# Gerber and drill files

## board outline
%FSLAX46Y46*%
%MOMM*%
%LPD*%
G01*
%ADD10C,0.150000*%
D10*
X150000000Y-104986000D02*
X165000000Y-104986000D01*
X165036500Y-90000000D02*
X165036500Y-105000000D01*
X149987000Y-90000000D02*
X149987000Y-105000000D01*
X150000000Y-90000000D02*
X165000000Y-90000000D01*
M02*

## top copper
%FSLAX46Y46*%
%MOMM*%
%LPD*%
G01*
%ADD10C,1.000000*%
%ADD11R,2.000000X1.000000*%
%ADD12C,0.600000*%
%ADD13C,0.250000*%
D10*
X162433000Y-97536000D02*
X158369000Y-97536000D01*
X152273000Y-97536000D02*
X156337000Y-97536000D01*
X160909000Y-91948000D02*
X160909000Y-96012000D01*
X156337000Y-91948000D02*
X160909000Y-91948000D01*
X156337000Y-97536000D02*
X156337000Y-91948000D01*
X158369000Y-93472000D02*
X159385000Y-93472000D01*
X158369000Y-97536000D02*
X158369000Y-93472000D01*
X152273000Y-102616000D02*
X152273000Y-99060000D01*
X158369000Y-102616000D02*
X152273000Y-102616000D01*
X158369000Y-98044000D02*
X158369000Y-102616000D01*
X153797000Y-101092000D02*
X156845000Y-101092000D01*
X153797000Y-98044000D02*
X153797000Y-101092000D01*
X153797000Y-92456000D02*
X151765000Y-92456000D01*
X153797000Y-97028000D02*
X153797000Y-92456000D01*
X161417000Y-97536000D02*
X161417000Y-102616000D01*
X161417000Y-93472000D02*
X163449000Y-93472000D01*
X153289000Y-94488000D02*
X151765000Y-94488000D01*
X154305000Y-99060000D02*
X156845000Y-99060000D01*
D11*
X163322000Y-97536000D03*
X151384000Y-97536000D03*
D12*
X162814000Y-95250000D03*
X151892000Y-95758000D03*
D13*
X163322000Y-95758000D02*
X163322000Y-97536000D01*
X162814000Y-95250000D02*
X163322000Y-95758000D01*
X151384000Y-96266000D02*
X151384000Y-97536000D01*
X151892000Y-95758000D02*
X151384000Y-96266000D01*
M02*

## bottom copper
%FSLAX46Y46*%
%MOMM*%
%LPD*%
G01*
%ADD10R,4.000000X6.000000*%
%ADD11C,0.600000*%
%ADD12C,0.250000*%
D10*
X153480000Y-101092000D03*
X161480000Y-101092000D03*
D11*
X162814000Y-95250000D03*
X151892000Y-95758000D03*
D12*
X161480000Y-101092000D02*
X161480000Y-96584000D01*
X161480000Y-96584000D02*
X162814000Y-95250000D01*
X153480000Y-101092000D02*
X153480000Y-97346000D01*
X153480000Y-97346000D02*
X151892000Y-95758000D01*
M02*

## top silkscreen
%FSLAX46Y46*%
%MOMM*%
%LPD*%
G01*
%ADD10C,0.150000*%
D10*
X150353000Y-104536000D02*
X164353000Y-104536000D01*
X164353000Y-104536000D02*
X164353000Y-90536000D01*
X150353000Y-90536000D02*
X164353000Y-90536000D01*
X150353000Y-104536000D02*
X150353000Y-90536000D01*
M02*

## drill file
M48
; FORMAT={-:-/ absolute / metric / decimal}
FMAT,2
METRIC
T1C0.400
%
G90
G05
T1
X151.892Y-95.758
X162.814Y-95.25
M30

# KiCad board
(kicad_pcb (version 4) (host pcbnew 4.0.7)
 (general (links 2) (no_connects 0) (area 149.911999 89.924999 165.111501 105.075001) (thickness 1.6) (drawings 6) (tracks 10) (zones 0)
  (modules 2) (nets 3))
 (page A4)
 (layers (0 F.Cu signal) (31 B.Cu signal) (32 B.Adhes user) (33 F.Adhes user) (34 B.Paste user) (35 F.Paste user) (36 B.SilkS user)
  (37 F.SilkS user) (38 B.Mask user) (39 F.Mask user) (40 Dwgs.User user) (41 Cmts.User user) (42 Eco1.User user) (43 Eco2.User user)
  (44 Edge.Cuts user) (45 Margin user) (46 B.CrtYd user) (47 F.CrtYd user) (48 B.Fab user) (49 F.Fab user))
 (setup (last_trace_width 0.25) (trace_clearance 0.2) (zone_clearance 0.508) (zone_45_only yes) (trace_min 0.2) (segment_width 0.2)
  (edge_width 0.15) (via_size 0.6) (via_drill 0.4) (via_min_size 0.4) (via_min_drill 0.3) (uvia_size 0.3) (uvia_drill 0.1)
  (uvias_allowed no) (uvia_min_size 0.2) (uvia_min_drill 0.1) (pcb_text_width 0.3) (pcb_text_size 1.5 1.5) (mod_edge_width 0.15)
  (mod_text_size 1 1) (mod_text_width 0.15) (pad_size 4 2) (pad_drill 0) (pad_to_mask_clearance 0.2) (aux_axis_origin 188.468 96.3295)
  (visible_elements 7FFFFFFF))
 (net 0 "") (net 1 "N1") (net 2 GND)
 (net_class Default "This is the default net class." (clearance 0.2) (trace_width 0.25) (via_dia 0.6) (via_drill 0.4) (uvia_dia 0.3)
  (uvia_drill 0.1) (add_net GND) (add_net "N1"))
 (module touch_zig (layer F.Cu) (at 157.353 97.536)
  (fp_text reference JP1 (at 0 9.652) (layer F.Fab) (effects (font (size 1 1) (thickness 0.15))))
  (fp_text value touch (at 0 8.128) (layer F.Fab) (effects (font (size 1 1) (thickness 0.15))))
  (fp_line (start 5.08 0) (end 1.016 0) (layer F.Cu) (width 1))
  (fp_line (start -5.08 0) (end -1.016 0) (layer F.Cu) (width 1))
  (fp_line (start 3.556 -5.588) (end 3.556 -1.524) (layer F.Cu) (width 1))
  (fp_line (start -1.016 -5.588) (end 3.556 -5.588) (layer F.Cu) (width 1))
  (fp_line (start -1.016 0) (end -1.016 -5.588) (layer F.Cu) (width 1))
  (fp_line (start 1.016 -4.064) (end 2.032 -4.064) (layer F.Cu) (width 1))
  (fp_line (start 1.016 0) (end 1.016 -4.064) (layer F.Cu) (width 1))
  (fp_line (start -5.08 5.08) (end -5.08 1.524) (layer F.Cu) (width 1))
  (fp_line (start 1.016 5.08) (end -5.08 5.08) (layer F.Cu) (width 1))
  (fp_line (start 1.016 0.508) (end 1.016 5.08) (layer F.Cu) (width 1))
  (fp_line (start -3.556 3.556) (end -0.508 3.556) (layer F.Cu) (width 1))
  (fp_line (start -3.556 0.508) (end -3.556 3.556) (layer F.Cu) (width 1))
  (fp_line (start -3.556 -5.08) (end -5.588 -5.08) (layer F.Cu) (width 1))
  (fp_line (start -3.556 -0.508) (end -3.556 -5.08) (layer F.Cu) (width 1))
  (fp_line (start 4.064 0) (end 4.064 5.08) (layer F.Cu) (width 1))
  (fp_line (start 4.064 -4.064) (end 6.096 -4.064) (layer F.Cu) (width 1))
  (fp_line (start -4.064 -3.048) (end -5.588 -3.048) (layer F.Cu) (width 1))
  (fp_line (start -3.048 1.524) (end -0.508 1.524) (layer F.Cu) (width 1))
  (fp_line (start -7 7) (end 7 7) (layer F.SilkS) (width 0.15))
  (fp_line (start 7 7) (end 7 -7) (layer F.SilkS) (width 0.15))
  (fp_line (start -7 -7) (end 7 -7) (layer F.SilkS) (width 0.15))
  (fp_line (start -7 7) (end -7 -7) (layer F.SilkS) (width 0.15))
  (pad 2 smd rect (at 5.969 0) (size 2 1) (layers F.Cu F.Paste F.Mask) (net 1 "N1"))
  (pad 1 smd rect (at -5.969 0) (size 2 1) (layers F.Cu F.Paste F.Mask) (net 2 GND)))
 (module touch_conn (layer B.Cu) (at 157.48 101.092 90)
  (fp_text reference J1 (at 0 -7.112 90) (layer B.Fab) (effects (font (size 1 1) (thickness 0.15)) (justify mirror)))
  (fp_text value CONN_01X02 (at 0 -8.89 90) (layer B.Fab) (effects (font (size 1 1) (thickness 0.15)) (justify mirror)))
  (pad 2 smd rect (at 0 -4 90) (size 6 4) (layers B.Cu B.Paste B.Mask) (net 2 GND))
  (pad 1 smd rect (at 0 4 90) (size 6 4) (layers B.Cu B.Paste B.Mask) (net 1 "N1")))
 (gr_line (start 150 104.986) (end 165 104.986) (angle 90) (layer Edge.Cuts) (width 0.15))
 (gr_line (start 165.0365 90) (end 165.0365 105) (angle 90) (layer Edge.Cuts) (width 0.15))
 (gr_line (start 149.987 90) (end 149.987 105) (angle 90) (layer Edge.Cuts) (width 0.15))
 (gr_line (start 150 90) (end 165 90) (angle 90) (layer Edge.Cuts) (width 0.15))
 (segment (start 161.48 101.092) (end 161.48 96.584) (width 0.25) (layer B.Cu) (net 1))
 (segment (start 163.322 95.758) (end 163.322 97.536) (width 0.25) (layer F.Cu) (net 1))
 (segment (start 162.814 95.25) (end 163.322 95.758) (width 0.25) (layer F.Cu) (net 1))
 (via (at 162.814 95.25) (size 0.6) (drill 0.4) (layers F.Cu B.Cu) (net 1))
 (segment (start 161.48 96.584) (end 162.814 95.25) (width 0.25) (layer B.Cu) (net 1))
 (segment (start 153.48 101.092) (end 153.48 97.346) (width 0.25) (layer B.Cu) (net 2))
 (segment (start 151.384 96.266) (end 151.384 97.536) (width 0.25) (layer F.Cu) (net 2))
 (segment (start 151.892 95.758) (end 151.384 96.266) (width 0.25) (layer F.Cu) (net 2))
 (via (at 151.892 95.758) (size 0.6) (drill 0.4) (layers F.Cu B.Cu) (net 2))
 (segment (start 153.48 97.346) (end 151.892 95.758) (width 0.25) (layer B.Cu) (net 2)))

